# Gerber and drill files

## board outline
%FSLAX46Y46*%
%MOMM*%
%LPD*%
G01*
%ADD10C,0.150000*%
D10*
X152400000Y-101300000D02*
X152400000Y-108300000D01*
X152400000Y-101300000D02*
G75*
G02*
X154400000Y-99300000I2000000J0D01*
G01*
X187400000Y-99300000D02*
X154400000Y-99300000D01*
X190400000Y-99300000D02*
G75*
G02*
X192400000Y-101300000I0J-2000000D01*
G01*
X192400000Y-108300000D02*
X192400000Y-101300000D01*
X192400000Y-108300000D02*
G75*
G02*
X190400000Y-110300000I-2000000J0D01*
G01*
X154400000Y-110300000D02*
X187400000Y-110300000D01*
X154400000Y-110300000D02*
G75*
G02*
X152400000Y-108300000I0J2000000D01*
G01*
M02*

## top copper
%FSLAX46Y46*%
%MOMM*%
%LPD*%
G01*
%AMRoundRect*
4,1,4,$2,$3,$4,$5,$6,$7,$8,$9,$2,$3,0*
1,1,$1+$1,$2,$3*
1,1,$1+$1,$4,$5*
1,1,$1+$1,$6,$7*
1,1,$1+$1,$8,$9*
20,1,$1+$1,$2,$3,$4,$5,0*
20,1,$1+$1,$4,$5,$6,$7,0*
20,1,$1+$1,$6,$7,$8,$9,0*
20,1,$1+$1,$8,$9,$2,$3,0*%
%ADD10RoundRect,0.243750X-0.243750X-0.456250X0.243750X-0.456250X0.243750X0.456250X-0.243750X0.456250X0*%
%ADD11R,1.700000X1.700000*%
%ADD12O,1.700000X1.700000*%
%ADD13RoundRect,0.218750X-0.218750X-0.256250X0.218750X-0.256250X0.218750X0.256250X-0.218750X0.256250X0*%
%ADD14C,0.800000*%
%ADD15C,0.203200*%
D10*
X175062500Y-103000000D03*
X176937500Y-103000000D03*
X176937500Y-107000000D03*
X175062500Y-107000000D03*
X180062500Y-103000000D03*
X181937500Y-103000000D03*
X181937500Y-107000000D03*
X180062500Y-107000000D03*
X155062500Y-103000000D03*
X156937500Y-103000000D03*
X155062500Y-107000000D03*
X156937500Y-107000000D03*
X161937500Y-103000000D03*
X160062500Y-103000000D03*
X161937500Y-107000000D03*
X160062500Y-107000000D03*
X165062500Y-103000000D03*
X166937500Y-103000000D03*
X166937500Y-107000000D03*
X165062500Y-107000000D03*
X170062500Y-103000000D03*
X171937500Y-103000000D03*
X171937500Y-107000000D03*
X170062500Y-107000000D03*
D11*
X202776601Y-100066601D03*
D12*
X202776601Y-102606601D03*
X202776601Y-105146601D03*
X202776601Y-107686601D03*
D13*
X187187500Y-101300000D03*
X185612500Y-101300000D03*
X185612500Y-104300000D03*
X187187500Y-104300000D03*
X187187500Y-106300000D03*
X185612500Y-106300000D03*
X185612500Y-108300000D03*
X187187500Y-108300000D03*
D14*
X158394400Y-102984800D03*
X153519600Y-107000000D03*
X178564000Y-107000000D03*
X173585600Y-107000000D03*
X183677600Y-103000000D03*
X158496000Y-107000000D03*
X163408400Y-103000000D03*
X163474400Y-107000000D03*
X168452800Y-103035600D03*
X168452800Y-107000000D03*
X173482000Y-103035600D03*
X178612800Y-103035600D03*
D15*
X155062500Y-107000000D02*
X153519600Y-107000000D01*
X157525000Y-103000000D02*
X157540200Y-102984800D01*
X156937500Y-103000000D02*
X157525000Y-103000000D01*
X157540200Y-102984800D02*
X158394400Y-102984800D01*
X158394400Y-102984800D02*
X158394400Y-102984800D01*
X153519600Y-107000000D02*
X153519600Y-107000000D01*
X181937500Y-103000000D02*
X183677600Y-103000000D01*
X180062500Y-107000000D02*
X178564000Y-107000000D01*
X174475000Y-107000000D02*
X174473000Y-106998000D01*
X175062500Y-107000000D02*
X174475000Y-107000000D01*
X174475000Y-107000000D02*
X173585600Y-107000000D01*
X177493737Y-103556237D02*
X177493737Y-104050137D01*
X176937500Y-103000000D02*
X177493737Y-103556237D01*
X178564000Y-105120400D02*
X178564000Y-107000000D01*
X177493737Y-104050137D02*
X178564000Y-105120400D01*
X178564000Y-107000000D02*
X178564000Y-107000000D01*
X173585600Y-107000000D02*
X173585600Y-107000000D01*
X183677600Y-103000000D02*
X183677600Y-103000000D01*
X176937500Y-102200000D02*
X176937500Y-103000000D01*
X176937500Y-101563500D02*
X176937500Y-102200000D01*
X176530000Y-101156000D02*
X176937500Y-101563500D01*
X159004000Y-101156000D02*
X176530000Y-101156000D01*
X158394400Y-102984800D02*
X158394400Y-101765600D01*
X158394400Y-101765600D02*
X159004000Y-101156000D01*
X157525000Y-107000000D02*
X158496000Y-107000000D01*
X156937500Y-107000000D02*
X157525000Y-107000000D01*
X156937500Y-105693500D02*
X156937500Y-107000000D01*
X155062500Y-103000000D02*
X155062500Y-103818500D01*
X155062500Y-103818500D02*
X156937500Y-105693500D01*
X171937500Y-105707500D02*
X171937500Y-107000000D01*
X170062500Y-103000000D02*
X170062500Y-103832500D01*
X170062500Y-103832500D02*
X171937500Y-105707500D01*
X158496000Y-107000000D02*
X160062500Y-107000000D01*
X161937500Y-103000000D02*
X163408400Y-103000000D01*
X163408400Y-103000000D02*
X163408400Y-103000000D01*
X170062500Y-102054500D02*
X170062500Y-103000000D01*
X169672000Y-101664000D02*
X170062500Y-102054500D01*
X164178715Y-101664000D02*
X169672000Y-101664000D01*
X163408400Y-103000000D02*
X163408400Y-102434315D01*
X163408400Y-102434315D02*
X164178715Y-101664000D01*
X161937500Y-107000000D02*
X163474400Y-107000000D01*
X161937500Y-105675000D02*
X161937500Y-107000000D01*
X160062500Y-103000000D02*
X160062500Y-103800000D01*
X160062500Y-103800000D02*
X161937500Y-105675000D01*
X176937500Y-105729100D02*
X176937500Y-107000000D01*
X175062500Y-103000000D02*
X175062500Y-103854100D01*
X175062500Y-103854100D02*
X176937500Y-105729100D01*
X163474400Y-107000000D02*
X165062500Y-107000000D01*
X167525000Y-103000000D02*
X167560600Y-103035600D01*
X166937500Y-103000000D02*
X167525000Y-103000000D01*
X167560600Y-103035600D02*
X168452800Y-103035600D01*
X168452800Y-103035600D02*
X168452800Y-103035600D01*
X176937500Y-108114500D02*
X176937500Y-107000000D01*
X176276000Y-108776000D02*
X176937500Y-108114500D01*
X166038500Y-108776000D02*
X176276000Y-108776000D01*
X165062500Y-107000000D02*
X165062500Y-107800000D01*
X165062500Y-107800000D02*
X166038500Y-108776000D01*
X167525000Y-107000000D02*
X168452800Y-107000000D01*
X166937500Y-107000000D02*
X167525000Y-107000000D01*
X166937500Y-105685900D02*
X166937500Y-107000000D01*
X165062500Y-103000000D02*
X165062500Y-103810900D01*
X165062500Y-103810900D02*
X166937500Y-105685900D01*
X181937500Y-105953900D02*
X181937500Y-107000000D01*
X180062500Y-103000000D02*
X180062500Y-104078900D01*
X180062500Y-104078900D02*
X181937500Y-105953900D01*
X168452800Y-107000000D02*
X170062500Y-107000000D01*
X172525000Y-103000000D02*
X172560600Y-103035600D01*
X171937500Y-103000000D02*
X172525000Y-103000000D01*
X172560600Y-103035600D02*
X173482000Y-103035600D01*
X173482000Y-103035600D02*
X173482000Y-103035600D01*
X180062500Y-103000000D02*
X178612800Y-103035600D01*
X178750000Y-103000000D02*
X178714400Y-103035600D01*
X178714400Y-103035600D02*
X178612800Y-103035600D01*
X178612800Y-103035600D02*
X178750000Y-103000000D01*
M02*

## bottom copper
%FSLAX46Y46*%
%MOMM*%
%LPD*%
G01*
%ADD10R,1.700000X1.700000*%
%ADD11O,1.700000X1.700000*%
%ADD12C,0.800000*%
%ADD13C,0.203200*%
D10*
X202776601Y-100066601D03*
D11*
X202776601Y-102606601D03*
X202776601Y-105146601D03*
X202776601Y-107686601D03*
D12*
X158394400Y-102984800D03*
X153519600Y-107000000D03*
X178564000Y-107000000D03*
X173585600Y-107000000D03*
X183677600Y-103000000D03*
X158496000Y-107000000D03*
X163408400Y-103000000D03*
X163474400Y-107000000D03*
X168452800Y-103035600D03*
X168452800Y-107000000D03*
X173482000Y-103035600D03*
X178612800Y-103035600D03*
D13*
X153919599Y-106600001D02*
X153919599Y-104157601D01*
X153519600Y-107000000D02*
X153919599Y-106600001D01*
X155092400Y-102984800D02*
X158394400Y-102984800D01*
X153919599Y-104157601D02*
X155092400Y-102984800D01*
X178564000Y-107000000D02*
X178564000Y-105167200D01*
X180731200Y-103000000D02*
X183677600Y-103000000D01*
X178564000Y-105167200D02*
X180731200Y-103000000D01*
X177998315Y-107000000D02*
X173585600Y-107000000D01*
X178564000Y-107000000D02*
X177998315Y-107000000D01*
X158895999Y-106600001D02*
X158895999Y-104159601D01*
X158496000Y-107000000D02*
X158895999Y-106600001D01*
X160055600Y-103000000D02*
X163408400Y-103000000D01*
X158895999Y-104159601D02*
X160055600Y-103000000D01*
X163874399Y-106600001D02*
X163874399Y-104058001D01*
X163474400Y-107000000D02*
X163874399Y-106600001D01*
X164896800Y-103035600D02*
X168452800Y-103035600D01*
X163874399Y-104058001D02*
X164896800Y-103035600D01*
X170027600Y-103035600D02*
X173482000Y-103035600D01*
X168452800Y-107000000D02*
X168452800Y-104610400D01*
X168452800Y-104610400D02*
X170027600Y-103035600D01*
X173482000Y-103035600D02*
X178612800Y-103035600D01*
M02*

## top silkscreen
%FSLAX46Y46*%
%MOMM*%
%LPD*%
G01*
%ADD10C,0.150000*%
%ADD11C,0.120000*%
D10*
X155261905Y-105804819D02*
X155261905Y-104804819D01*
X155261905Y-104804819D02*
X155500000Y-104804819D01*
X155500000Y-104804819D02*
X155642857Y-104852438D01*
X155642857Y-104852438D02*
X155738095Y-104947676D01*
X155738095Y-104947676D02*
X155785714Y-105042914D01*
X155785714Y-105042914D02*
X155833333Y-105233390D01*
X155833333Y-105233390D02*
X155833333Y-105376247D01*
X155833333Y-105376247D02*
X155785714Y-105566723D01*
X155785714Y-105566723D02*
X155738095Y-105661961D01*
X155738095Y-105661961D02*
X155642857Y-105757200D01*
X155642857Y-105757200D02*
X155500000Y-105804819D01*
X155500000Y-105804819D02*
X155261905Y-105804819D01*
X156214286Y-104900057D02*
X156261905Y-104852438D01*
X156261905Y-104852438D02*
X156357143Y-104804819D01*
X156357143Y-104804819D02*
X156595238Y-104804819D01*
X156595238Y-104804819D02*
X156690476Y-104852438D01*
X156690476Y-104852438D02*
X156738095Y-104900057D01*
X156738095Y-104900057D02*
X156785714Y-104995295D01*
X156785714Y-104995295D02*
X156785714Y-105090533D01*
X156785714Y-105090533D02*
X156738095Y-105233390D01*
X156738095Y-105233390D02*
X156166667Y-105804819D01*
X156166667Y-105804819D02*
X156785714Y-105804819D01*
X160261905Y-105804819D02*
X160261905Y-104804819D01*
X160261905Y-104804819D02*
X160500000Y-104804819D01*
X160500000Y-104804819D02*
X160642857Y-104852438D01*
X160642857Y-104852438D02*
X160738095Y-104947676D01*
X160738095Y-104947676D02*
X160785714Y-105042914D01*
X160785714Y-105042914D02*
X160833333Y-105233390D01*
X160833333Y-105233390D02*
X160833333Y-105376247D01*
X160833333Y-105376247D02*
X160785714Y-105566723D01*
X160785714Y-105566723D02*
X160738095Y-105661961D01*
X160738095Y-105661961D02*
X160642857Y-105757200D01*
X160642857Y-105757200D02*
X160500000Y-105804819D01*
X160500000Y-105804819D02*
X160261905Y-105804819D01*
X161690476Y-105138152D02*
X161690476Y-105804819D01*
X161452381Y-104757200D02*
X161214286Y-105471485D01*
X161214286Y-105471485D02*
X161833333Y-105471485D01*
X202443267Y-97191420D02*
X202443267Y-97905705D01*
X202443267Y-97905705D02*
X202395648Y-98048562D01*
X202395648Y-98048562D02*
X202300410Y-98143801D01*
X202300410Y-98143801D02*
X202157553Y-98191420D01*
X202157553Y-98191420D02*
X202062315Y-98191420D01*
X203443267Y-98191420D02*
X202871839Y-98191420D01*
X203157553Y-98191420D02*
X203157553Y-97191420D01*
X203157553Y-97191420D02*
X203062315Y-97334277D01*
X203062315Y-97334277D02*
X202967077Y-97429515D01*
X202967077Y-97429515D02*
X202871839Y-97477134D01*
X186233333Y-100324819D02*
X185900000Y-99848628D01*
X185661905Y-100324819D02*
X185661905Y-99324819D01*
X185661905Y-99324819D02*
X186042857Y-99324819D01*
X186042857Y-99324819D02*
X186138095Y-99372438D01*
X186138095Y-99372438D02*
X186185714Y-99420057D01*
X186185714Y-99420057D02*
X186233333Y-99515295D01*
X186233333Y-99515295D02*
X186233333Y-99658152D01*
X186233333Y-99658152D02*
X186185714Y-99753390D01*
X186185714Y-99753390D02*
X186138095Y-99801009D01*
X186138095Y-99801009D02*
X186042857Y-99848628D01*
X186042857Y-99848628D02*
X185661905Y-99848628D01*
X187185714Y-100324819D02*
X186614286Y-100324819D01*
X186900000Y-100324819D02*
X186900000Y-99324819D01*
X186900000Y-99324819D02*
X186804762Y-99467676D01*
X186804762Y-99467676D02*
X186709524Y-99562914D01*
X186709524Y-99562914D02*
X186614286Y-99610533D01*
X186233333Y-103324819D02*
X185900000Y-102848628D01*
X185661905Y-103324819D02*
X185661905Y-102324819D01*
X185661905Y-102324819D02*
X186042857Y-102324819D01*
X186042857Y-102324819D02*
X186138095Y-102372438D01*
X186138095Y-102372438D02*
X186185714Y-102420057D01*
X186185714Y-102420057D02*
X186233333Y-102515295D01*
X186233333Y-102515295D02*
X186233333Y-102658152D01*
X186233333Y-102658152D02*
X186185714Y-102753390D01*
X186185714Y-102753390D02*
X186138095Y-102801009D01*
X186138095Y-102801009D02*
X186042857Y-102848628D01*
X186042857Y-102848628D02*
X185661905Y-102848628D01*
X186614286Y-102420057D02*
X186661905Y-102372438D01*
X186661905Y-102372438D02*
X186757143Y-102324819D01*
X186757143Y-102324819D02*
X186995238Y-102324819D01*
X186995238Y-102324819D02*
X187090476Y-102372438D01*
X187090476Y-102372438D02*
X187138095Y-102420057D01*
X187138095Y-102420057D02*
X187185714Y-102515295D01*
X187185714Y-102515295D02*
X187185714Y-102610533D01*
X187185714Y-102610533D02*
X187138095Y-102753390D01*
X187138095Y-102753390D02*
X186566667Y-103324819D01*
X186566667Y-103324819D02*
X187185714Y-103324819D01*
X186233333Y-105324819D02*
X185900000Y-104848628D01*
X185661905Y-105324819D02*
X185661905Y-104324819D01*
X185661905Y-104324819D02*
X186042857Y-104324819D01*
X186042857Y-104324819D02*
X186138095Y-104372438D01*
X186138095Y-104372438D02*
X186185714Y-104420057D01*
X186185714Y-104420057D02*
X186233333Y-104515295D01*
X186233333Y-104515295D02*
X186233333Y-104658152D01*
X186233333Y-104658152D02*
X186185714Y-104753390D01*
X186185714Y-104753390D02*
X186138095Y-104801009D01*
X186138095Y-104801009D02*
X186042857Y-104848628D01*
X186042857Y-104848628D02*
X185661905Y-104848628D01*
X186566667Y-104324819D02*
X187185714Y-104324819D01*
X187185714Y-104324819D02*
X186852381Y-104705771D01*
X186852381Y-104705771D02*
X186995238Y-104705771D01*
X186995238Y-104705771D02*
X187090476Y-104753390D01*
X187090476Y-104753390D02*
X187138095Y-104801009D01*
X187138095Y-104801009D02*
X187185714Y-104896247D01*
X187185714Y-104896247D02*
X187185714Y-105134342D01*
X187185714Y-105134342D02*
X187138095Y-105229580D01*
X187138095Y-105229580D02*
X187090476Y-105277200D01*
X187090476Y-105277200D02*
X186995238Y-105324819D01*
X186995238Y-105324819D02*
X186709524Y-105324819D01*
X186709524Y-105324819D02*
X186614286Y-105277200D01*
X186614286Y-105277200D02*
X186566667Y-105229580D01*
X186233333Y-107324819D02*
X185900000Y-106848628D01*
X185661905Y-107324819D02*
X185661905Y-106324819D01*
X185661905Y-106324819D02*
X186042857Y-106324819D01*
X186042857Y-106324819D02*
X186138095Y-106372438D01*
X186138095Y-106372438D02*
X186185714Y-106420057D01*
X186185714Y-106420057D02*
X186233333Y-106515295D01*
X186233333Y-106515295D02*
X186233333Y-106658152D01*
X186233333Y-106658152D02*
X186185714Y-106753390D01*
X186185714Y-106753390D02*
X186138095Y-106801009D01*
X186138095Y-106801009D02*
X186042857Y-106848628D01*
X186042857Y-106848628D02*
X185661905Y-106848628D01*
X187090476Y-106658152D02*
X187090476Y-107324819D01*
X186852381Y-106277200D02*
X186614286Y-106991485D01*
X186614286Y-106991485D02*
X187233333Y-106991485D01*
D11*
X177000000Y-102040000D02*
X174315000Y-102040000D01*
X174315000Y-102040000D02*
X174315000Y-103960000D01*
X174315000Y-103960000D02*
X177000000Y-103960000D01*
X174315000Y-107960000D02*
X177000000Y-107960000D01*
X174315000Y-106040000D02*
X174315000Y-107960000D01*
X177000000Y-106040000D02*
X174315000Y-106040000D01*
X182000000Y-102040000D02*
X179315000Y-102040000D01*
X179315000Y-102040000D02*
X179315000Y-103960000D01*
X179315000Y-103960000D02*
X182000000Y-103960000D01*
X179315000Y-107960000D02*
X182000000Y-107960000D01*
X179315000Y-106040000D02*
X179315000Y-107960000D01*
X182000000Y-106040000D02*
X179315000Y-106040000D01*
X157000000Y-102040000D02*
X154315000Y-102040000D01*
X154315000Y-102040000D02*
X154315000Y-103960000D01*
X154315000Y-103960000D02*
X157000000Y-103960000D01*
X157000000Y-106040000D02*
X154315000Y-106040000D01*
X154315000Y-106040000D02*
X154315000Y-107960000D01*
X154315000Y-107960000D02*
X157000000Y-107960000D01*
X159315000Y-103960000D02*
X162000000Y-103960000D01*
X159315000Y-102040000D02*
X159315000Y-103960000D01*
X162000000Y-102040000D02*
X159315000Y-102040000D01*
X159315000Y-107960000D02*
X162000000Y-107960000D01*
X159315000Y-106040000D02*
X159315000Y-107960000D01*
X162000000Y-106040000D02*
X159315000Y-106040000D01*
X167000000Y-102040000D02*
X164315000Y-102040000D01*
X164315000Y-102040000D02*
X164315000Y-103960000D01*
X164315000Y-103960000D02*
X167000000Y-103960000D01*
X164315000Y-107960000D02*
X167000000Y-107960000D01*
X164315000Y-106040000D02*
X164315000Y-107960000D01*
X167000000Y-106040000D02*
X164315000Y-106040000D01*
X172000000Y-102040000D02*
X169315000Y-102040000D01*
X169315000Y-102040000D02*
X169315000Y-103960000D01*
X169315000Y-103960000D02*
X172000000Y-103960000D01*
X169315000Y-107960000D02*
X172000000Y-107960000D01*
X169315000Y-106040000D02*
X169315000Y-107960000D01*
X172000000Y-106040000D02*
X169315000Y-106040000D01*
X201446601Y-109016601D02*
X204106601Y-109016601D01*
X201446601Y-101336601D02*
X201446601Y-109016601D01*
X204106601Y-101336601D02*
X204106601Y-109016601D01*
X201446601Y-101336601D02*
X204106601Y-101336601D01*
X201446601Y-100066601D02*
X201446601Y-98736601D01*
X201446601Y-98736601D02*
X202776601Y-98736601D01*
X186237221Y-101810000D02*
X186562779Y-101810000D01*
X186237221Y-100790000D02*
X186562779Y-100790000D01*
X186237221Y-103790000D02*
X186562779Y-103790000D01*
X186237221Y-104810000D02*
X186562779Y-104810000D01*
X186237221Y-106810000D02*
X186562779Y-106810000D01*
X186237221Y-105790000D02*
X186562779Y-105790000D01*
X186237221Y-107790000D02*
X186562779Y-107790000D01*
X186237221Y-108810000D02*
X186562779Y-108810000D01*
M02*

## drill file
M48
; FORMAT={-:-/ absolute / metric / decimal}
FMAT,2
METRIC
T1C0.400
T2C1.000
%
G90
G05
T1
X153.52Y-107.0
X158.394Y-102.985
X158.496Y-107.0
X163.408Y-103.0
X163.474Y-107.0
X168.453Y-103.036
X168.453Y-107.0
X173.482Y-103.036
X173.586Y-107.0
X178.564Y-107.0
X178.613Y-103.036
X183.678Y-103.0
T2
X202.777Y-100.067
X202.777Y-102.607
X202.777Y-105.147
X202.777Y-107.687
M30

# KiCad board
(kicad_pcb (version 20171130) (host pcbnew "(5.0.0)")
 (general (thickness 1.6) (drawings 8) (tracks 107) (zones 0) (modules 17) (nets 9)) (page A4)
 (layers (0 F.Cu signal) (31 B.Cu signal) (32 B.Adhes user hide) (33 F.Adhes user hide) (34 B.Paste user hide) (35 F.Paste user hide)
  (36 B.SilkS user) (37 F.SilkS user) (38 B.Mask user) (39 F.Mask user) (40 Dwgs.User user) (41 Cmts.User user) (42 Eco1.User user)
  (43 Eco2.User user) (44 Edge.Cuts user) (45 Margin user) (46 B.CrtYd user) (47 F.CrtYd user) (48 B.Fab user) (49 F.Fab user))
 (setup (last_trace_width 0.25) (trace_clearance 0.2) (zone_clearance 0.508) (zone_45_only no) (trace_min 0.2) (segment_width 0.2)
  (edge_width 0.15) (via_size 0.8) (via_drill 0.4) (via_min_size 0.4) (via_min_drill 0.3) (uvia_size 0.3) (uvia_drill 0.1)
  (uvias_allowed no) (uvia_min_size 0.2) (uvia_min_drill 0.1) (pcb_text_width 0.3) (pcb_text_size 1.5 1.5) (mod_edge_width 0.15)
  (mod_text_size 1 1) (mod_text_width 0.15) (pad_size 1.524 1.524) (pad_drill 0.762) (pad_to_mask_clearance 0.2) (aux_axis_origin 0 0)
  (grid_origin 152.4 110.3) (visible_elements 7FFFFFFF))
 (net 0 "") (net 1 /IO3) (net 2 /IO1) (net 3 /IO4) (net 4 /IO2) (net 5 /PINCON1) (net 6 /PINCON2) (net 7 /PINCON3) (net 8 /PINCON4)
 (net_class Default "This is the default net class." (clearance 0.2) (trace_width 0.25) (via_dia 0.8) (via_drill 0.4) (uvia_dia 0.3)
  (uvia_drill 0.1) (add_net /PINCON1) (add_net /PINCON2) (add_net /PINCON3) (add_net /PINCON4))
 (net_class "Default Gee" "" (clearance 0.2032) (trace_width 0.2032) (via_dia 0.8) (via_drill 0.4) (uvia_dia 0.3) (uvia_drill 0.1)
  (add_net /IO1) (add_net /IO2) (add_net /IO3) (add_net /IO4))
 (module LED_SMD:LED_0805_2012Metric (layer F.Cu) (at 176 103)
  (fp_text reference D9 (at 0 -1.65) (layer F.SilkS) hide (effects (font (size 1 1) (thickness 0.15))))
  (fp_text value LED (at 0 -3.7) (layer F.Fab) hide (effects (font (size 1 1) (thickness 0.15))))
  (fp_line (start 1 -0.96) (end -1.685 -0.96) (layer F.SilkS) (width 0.12))
  (fp_line (start -1.685 -0.96) (end -1.685 0.96) (layer F.SilkS) (width 0.12))
  (fp_line (start -1.685 0.96) (end 1 0.96) (layer F.SilkS) (width 0.12))
  (pad 1 smd roundrect (at -0.9375 0) (size 0.975 1.4) (layers F.Cu F.Paste F.Mask) (roundrect_rratio 0.25) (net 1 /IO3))
  (pad 2 smd roundrect (at 0.9375 0) (size 0.975 1.4) (layers F.Cu F.Paste F.Mask) (roundrect_rratio 0.25) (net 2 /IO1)))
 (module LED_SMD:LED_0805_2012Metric (layer F.Cu) (at 176 107)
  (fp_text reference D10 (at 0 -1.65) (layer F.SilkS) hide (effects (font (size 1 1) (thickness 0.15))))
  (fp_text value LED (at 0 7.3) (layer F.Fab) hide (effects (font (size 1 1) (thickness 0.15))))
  (fp_line (start -1.685 0.96) (end 1 0.96) (layer F.SilkS) (width 0.12))
  (fp_line (start -1.685 -0.96) (end -1.685 0.96) (layer F.SilkS) (width 0.12))
  (fp_line (start 1 -0.96) (end -1.685 -0.96) (layer F.SilkS) (width 0.12))
  (pad 2 smd roundrect (at 0.9375 0) (size 0.975 1.4) (layers F.Cu F.Paste F.Mask) (roundrect_rratio 0.25) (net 1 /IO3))
  (pad 1 smd roundrect (at -0.9375 0) (size 0.975 1.4) (layers F.Cu F.Paste F.Mask) (roundrect_rratio 0.25) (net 2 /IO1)))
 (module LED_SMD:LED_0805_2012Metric (layer F.Cu) (at 181 103)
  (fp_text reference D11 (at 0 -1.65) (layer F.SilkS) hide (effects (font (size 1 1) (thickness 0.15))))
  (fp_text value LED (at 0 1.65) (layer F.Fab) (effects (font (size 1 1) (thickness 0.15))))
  (fp_line (start 1 -0.96) (end -1.685 -0.96) (layer F.SilkS) (width 0.12))
  (fp_line (start -1.685 -0.96) (end -1.685 0.96) (layer F.SilkS) (width 0.12))
  (fp_line (start -1.685 0.96) (end 1 0.96) (layer F.SilkS) (width 0.12))
  (pad 1 smd roundrect (at -0.9375 0) (size 0.975 1.4) (layers F.Cu F.Paste F.Mask) (roundrect_rratio 0.25) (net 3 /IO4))
  (pad 2 smd roundrect (at 0.9375 0) (size 0.975 1.4) (layers F.Cu F.Paste F.Mask) (roundrect_rratio 0.25) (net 2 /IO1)))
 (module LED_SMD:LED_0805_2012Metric (layer F.Cu) (at 181 107)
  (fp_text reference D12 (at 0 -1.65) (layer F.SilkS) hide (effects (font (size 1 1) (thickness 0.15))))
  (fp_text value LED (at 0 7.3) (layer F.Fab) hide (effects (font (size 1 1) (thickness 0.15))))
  (fp_line (start -1.685 0.96) (end 1 0.96) (layer F.SilkS) (width 0.12))
  (fp_line (start -1.685 -0.96) (end -1.685 0.96) (layer F.SilkS) (width 0.12))
  (fp_line (start 1 -0.96) (end -1.685 -0.96) (layer F.SilkS) (width 0.12))
  (pad 2 smd roundrect (at 0.9375 0) (size 0.975 1.4) (layers F.Cu F.Paste F.Mask) (roundrect_rratio 0.25) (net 3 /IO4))
  (pad 1 smd roundrect (at -0.9375 0) (size 0.975 1.4) (layers F.Cu F.Paste F.Mask) (roundrect_rratio 0.25) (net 2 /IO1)))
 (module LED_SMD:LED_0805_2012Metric (layer F.Cu) (at 156 103)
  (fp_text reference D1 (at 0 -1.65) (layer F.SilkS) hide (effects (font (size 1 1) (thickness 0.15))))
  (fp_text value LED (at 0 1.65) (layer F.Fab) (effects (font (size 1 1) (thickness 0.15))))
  (fp_line (start 1 -0.96) (end -1.685 -0.96) (layer F.SilkS) (width 0.12))
  (fp_line (start -1.685 -0.96) (end -1.685 0.96) (layer F.SilkS) (width 0.12))
  (fp_line (start -1.685 0.96) (end 1 0.96) (layer F.SilkS) (width 0.12))
  (pad 1 smd roundrect (at -0.9375 0) (size 0.975 1.4) (layers F.Cu F.Paste F.Mask) (roundrect_rratio 0.25) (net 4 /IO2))
  (pad 2 smd roundrect (at 0.9375 0) (size 0.975 1.4) (layers F.Cu F.Paste F.Mask) (roundrect_rratio 0.25) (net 2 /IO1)))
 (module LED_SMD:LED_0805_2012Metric (layer F.Cu) (at 156 107)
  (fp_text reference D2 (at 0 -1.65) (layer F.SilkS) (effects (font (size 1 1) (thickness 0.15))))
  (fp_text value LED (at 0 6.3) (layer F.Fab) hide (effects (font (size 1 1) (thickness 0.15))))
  (fp_line (start 1 -0.96) (end -1.685 -0.96) (layer F.SilkS) (width 0.12))
  (fp_line (start -1.685 -0.96) (end -1.685 0.96) (layer F.SilkS) (width 0.12))
  (fp_line (start -1.685 0.96) (end 1 0.96) (layer F.SilkS) (width 0.12))
  (pad 1 smd roundrect (at -0.9375 0) (size 0.975 1.4) (layers F.Cu F.Paste F.Mask) (roundrect_rratio 0.25) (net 2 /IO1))
  (pad 2 smd roundrect (at 0.9375 0) (size 0.975 1.4) (layers F.Cu F.Paste F.Mask) (roundrect_rratio 0.25) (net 4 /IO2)))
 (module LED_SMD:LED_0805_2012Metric (layer F.Cu) (at 161 103)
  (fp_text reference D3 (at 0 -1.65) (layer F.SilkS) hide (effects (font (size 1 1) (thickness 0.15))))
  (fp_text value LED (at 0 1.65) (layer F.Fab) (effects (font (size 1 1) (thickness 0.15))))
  (fp_line (start -1.685 0.96) (end 1 0.96) (layer F.SilkS) (width 0.12))
  (fp_line (start -1.685 -0.96) (end -1.685 0.96) (layer F.SilkS) (width 0.12))
  (fp_line (start 1 -0.96) (end -1.685 -0.96) (layer F.SilkS) (width 0.12))
  (pad 2 smd roundrect (at 0.9375 0) (size 0.975 1.4) (layers F.Cu F.Paste F.Mask) (roundrect_rratio 0.25) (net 4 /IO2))
  (pad 1 smd roundrect (at -0.9375 0) (size 0.975 1.4) (layers F.Cu F.Paste F.Mask) (roundrect_rratio 0.25) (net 1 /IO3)))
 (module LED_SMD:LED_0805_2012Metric (layer F.Cu) (at 161 107)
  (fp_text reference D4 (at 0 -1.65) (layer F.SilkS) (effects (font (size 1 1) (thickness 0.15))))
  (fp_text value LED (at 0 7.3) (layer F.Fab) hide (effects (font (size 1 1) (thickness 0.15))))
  (fp_line (start -1.685 0.96) (end 1 0.96) (layer F.SilkS) (width 0.12))
  (fp_line (start -1.685 -0.96) (end -1.685 0.96) (layer F.SilkS) (width 0.12))
  (fp_line (start 1 -0.96) (end -1.685 -0.96) (layer F.SilkS) (width 0.12))
  (pad 2 smd roundrect (at 0.9375 0) (size 0.975 1.4) (layers F.Cu F.Paste F.Mask) (roundrect_rratio 0.25) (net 1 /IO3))
  (pad 1 smd roundrect (at -0.9375 0) (size 0.975 1.4) (layers F.Cu F.Paste F.Mask) (roundrect_rratio 0.25) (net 4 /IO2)))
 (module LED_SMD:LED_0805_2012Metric (layer F.Cu) (at 166 103)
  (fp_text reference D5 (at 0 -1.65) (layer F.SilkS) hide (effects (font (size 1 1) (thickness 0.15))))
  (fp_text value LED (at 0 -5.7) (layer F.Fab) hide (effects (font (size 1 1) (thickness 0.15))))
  (fp_line (start 1 -0.96) (end -1.685 -0.96) (layer F.SilkS) (width 0.12))
  (fp_line (start -1.685 -0.96) (end -1.685 0.96) (layer F.SilkS) (width 0.12))
  (fp_line (start -1.685 0.96) (end 1 0.96) (layer F.SilkS) (width 0.12))
  (pad 1 smd roundrect (at -0.9375 0) (size 0.975 1.4) (layers F.Cu F.Paste F.Mask) (roundrect_rratio 0.25) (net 3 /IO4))
  (pad 2 smd roundrect (at 0.9375 0) (size 0.975 1.4) (layers F.Cu F.Paste F.Mask) (roundrect_rratio 0.25) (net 1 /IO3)))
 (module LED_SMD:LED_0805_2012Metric (layer F.Cu) (at 166 107)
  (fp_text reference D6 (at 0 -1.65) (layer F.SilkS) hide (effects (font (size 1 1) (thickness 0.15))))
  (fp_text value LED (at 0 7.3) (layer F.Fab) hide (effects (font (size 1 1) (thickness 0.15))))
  (fp_line (start -1.685 0.96) (end 1 0.96) (layer F.SilkS) (width 0.12))
  (fp_line (start -1.685 -0.96) (end -1.685 0.96) (layer F.SilkS) (width 0.12))
  (fp_line (start 1 -0.96) (end -1.685 -0.96) (layer F.SilkS) (width 0.12))
  (pad 2 smd roundrect (at 0.9375 0) (size 0.975 1.4) (layers F.Cu F.Paste F.Mask) (roundrect_rratio 0.25) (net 3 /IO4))
  (pad 1 smd roundrect (at -0.9375 0) (size 0.975 1.4) (layers F.Cu F.Paste F.Mask) (roundrect_rratio 0.25) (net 1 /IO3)))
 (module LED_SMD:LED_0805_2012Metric (layer F.Cu) (at 171 103)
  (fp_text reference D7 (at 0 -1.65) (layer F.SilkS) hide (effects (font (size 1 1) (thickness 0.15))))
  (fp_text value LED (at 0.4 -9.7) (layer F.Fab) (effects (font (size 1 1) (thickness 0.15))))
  (fp_line (start 1 -0.96) (end -1.685 -0.96) (layer F.SilkS) (width 0.12))
  (fp_line (start -1.685 -0.96) (end -1.685 0.96) (layer F.SilkS) (width 0.12))
  (fp_line (start -1.685 0.96) (end 1 0.96) (layer F.SilkS) (width 0.12))
  (pad 1 smd roundrect (at -0.9375 0) (size 0.975 1.4) (layers F.Cu F.Paste F.Mask) (roundrect_rratio 0.25) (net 4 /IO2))
  (pad 2 smd roundrect (at 0.9375 0) (size 0.975 1.4) (layers F.Cu F.Paste F.Mask) (roundrect_rratio 0.25) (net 3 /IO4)))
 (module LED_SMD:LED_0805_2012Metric (layer F.Cu) (at 171 107)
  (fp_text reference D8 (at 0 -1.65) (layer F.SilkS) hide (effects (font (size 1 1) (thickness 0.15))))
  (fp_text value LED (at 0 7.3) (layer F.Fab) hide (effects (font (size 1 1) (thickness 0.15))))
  (fp_line (start -1.685 0.96) (end 1 0.96) (layer F.SilkS) (width 0.12))
  (fp_line (start -1.685 -0.96) (end -1.685 0.96) (layer F.SilkS) (width 0.12))
  (fp_line (start 1 -0.96) (end -1.685 -0.96) (layer F.SilkS) (width 0.12))
  (pad 2 smd roundrect (at 0.9375 0) (size 0.975 1.4) (layers F.Cu F.Paste F.Mask) (roundrect_rratio 0.25) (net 4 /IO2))
  (pad 1 smd roundrect (at -0.9375 0) (size 0.975 1.4) (layers F.Cu F.Paste F.Mask) (roundrect_rratio 0.25) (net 3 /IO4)))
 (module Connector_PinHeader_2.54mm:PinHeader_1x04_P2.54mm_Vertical (layer F.Cu) (at 202.776601 100.066601)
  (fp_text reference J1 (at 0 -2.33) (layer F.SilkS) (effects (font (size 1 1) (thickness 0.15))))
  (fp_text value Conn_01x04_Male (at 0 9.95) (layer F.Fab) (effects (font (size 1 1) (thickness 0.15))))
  (fp_line (start -1.33 8.95) (end 1.33 8.95) (layer F.SilkS) (width 0.12))
  (fp_line (start -1.33 1.27) (end -1.33 8.95) (layer F.SilkS) (width 0.12))
  (fp_line (start 1.33 1.27) (end 1.33 8.95) (layer F.SilkS) (width 0.12))
  (fp_line (start -1.33 1.27) (end 1.33 1.27) (layer F.SilkS) (width 0.12))
  (fp_line (start -1.33 0) (end -1.33 -1.33) (layer F.SilkS) (width 0.12))
  (fp_line (start -1.33 -1.33) (end 0 -1.33) (layer F.SilkS) (width 0.12))
  (pad 1 thru_hole rect (at 0 0) (size 1.7 1.7) (drill 1) (layers *.Cu *.Mask) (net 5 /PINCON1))
  (pad 2 thru_hole oval (at 0 2.54) (size 1.7 1.7) (drill 1) (layers *.Cu *.Mask) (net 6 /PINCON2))
  (pad 3 thru_hole oval (at 0 5.08) (size 1.7 1.7) (drill 1) (layers *.Cu *.Mask) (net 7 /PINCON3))
  (pad 4 thru_hole oval (at 0 7.62) (size 1.7 1.7) (drill 1) (layers *.Cu *.Mask) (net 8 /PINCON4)))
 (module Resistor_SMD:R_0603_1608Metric (layer F.Cu) (at 186.4 101.3)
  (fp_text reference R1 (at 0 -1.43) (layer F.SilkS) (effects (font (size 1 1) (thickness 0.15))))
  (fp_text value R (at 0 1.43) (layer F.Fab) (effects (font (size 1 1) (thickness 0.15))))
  (fp_line (start -0.162779 0.51) (end 0.162779 0.51) (layer F.SilkS) (width 0.12))
  (fp_line (start -0.162779 -0.51) (end 0.162779 -0.51) (layer F.SilkS) (width 0.12))
  (pad 2 smd roundrect (at 0.7875 0) (size 0.875 0.95) (layers F.Cu F.Paste F.Mask) (roundrect_rratio 0.25) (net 2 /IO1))
  (pad 1 smd roundrect (at -0.7875 0) (size 0.875 0.95) (layers F.Cu F.Paste F.Mask) (roundrect_rratio 0.25) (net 5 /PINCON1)))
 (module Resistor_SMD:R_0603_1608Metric (layer F.Cu) (at 186.4 104.3)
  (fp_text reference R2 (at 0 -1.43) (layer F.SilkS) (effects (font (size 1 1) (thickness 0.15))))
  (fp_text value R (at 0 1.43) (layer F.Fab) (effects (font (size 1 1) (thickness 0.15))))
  (fp_line (start -0.162779 -0.51) (end 0.162779 -0.51) (layer F.SilkS) (width 0.12))
  (fp_line (start -0.162779 0.51) (end 0.162779 0.51) (layer F.SilkS) (width 0.12))
  (pad 1 smd roundrect (at -0.7875 0) (size 0.875 0.95) (layers F.Cu F.Paste F.Mask) (roundrect_rratio 0.25) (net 6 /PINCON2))
  (pad 2 smd roundrect (at 0.7875 0) (size 0.875 0.95) (layers F.Cu F.Paste F.Mask) (roundrect_rratio 0.25) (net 4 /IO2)))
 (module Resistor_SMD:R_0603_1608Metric (layer F.Cu) (at 186.4 106.3)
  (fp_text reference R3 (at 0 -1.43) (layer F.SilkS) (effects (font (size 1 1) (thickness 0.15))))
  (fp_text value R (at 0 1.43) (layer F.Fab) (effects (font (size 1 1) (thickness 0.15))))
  (fp_line (start -0.162779 0.51) (end 0.162779 0.51) (layer F.SilkS) (width 0.12))
  (fp_line (start -0.162779 -0.51) (end 0.162779 -0.51) (layer F.SilkS) (width 0.12))
  (pad 2 smd roundrect (at 0.7875 0) (size 0.875 0.95) (layers F.Cu F.Paste F.Mask) (roundrect_rratio 0.25) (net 1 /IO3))
  (pad 1 smd roundrect (at -0.7875 0) (size 0.875 0.95) (layers F.Cu F.Paste F.Mask) (roundrect_rratio 0.25) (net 7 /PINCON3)))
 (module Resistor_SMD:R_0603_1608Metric (layer F.Cu) (at 186.4 108.3)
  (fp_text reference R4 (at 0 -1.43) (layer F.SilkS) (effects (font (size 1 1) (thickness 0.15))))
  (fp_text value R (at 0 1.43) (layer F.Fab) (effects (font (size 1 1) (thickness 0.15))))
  (fp_line (start -0.162779 -0.51) (end 0.162779 -0.51) (layer F.SilkS) (width 0.12))
  (fp_line (start -0.162779 0.51) (end 0.162779 0.51) (layer F.SilkS) (width 0.12))
  (pad 1 smd roundrect (at -0.7875 0) (size 0.875 0.95) (layers F.Cu F.Paste F.Mask) (roundrect_rratio 0.25) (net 8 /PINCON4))
  (pad 2 smd roundrect (at 0.7875 0) (size 0.875 0.95) (layers F.Cu F.Paste F.Mask) (roundrect_rratio 0.25) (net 3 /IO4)))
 (gr_line (start 152.4 101.3) (end 152.4 108.3) (layer Edge.Cuts) (width 0.15))
 (gr_arc (start 154.4 101.3) (end 154.4 99.3) (angle -90) (layer Edge.Cuts) (width 0.15))
 (gr_line (start 187.4 99.3) (end 154.4 99.3) (layer Edge.Cuts) (width 0.15))
 (gr_arc (start 190.4 101.3) (end 192.4 101.3) (angle -90) (layer Edge.Cuts) (width 0.15))
 (gr_line (start 192.4 108.3) (end 192.4 101.3) (layer Edge.Cuts) (width 0.15))
 (gr_arc (start 190.4 108.3) (end 190.4 110.3) (angle -90) (layer Edge.Cuts) (width 0.15))
 (gr_line (start 154.4 110.3) (end 187.4 110.3) (layer Edge.Cuts) (width 0.15))
 (gr_arc (start 154.4 108.3) (end 152.4 108.3) (angle -90) (layer Edge.Cuts) (width 0.15))
 (segment (start 155.0625 107) (end 153.5196 107) (width 0.2032) (layer F.Cu) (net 2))
 (segment (start 157.525 103) (end 157.5402 102.9848) (width 0.2032) (layer F.Cu) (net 2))
 (segment (start 156.9375 103) (end 157.525 103) (width 0.2032) (layer F.Cu) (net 2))
 (segment (start 157.5402 102.9848) (end 158.3944 102.9848) (width 0.2032) (layer F.Cu) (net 2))
 (segment (start 158.3944 102.9848) (end 158.3944 102.9848) (width 0.2032) (layer F.Cu) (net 2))
 (via (at 158.3944 102.9848) (size 0.8) (drill 0.4) (layers F.Cu B.Cu) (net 2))
 (segment (start 153.5196 107) (end 153.5196 107) (width 0.2032) (layer F.Cu) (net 2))
 (via (at 153.5196 107) (size 0.8) (drill 0.4) (layers F.Cu B.Cu) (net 2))
 (segment (start 153.919599 106.600001) (end 153.919599 104.157601) (width 0.2032) (layer B.Cu) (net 2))
 (segment (start 153.5196 107) (end 153.919599 106.600001) (width 0.2032) (layer B.Cu) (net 2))
 (segment (start 155.0924 102.9848) (end 158.3944 102.9848) (width 0.2032) (layer B.Cu) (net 2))
 (segment (start 153.919599 104.157601) (end 155.0924 102.9848) (width 0.2032) (layer B.Cu) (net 2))
 (segment (start 181.9375 103) (end 183.6776 103) (width 0.2032) (layer F.Cu) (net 2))
 (segment (start 180.0625 107) (end 178.564 107) (width 0.2032) (layer F.Cu) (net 2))
 (segment (start 174.475 107) (end 174.473 106.998) (width 0.2032) (layer F.Cu) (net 2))
 (segment (start 175.0625 107) (end 174.475 107) (width 0.2032) (layer F.Cu) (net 2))
 (segment (start 174.475 107) (end 173.5856 107) (width 0.2032) (layer F.Cu) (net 2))
 (segment (start 177.493737 103.556237) (end 177.493737 104.050137) (width 0.2032) (layer F.Cu) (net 2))
 (segment (start 176.9375 103) (end 177.493737 103.556237) (width 0.2032) (layer F.Cu) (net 2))
 (segment (start 178.564 105.1204) (end 178.564 107) (width 0.2032) (layer F.Cu) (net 2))
 (segment (start 177.493737 104.050137) (end 178.564 105.1204) (width 0.2032) (layer F.Cu) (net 2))
 (segment (start 178.564 107) (end 178.564 107) (width 0.2032) (layer F.Cu) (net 2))
 (via (at 178.564 107) (size 0.8) (drill 0.4) (layers F.Cu B.Cu) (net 2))
 (segment (start 173.5856 107) (end 173.5856 107) (width 0.2032) (layer F.Cu) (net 2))
 (via (at 173.5856 107) (size 0.8) (drill 0.4) (layers F.Cu B.Cu) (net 2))
 (segment (start 183.6776 103) (end 183.6776 103) (width 0.2032) (layer F.Cu) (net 2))
 (via (at 183.6776 103) (size 0.8) (drill 0.4) (layers F.Cu B.Cu) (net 2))
 (segment (start 178.564 107) (end 178.564 105.1672) (width 0.2032) (layer B.Cu) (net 2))
 (segment (start 180.7312 103) (end 183.6776 103) (width 0.2032) (layer B.Cu) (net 2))
 (segment (start 178.564 105.1672) (end 180.7312 103) (width 0.2032) (layer B.Cu) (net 2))
 (segment (start 176.9375 102.2) (end 176.9375 103) (width 0.2032) (layer F.Cu) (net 2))
 (segment (start 176.9375 101.5635) (end 176.9375 102.2) (width 0.2032) (layer F.Cu) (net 2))
 (segment (start 176.53 101.156) (end 176.9375 101.5635) (width 0.2032) (layer F.Cu) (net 2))
 (segment (start 159.004 101.156) (end 176.53 101.156) (width 0.2032) (layer F.Cu) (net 2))
 (segment (start 158.3944 102.9848) (end 158.3944 101.7656) (width 0.2032) (layer F.Cu) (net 2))
 (segment (start 158.3944 101.7656) (end 159.004 101.156) (width 0.2032) (layer F.Cu) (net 2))
 (segment (start 177.998315 107) (end 173.5856 107) (width 0.2032) (layer B.Cu) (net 2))
 (segment (start 178.564 107) (end 177.998315 107) (width 0.2032) (layer B.Cu) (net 2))
 (segment (start 157.525 107) (end 158.496 107) (width 0.2032) (layer F.Cu) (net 4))
 (segment (start 156.9375 107) (end 157.525 107) (width 0.2032) (layer F.Cu) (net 4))
 (segment (start 156.9375 105.6935) (end 156.9375 107) (width 0.2032) (layer F.Cu) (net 4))
 (segment (start 155.0625 103) (end 155.0625 103.8185) (width 0.2032) (layer F.Cu) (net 4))
 (segment (start 155.0625 103.8185) (end 156.9375 105.6935) (width 0.2032) (layer F.Cu) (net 4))
 (segment (start 171.9375 105.7075) (end 171.9375 107) (width 0.2032) (layer F.Cu) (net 4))
 (segment (start 170.0625 103) (end 170.0625 103.8325) (width 0.2032) (layer F.Cu) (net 4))
 (segment (start 170.0625 103.8325) (end 171.9375 105.7075) (width 0.2032) (layer F.Cu) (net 4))
 (segment (start 158.496 107) (end 160.0625 107) (width 0.2032) (layer F.Cu) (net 4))
 (via (at 158.496 107) (size 0.8) (drill 0.4) (layers F.Cu B.Cu) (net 4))
 (segment (start 161.9375 103) (end 163.4084 103) (width 0.2032) (layer F.Cu) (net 4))
 (segment (start 163.4084 103) (end 163.4084 103) (width 0.2032) (layer F.Cu) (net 4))
 (via (at 163.4084 103) (size 0.8) (drill 0.4) (layers F.Cu B.Cu) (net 4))
 (segment (start 158.895999 106.600001) (end 158.895999 104.159601) (width 0.2032) (layer B.Cu) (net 4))
 (segment (start 158.496 107) (end 158.895999 106.600001) (width 0.2032) (layer B.Cu) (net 4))
 (segment (start 160.0556 103) (end 163.4084 103) (width 0.2032) (layer B.Cu) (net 4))
 (segment (start 158.895999 104.159601) (end 160.0556 103) (width 0.2032) (layer B.Cu) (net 4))
 (segment (start 170.0625 102.0545) (end 170.0625 103) (width 0.2032) (layer F.Cu) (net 4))
 (segment (start 169.672 101.664) (end 170.0625 102.0545) (width 0.2032) (layer F.Cu) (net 4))
 (segment (start 164.178715 101.664) (end 169.672 101.664) (width 0.2032) (layer F.Cu) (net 4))
 (segment (start 163.4084 103) (end 163.4084 102.434315) (width 0.2032) (layer F.Cu) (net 4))
 (segment (start 163.4084 102.434315) (end 164.178715 101.664) (width 0.2032) (layer F.Cu) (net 4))
 (segment (start 161.9375 107) (end 163.4744 107) (width 0.2032) (layer F.Cu) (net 1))
 (segment (start 161.9375 105.675) (end 161.9375 107) (width 0.2032) (layer F.Cu) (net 1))
 (segment (start 160.0625 103) (end 160.0625 103.8) (width 0.2032) (layer F.Cu) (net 1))
 (segment (start 160.0625 103.8) (end 161.9375 105.675) (width 0.2032) (layer F.Cu) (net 1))
 (segment (start 176.9375 105.7291) (end 176.9375 107) (width 0.2032) (layer F.Cu) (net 1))
 (segment (start 175.0625 103) (end 175.0625 103.8541) (width 0.2032) (layer F.Cu) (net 1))
 (segment (start 175.0625 103.8541) (end 176.9375 105.7291) (width 0.2032) (layer F.Cu) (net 1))
 (segment (start 163.4744 107) (end 165.0625 107) (width 0.2032) (layer F.Cu) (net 1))
 (via (at 163.4744 107) (size 0.8) (drill 0.4) (layers F.Cu B.Cu) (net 1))
 (segment (start 167.525 103) (end 167.5606 103.0356) (width 0.2032) (layer F.Cu) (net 1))
 (segment (start 166.9375 103) (end 167.525 103) (width 0.2032) (layer F.Cu) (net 1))
 (segment (start 167.5606 103.0356) (end 168.4528 103.0356) (width 0.2032) (layer F.Cu) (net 1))
 (segment (start 168.4528 103.0356) (end 168.4528 103.0356) (width 0.2032) (layer F.Cu) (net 1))
 (via (at 168.4528 103.0356) (size 0.8) (drill 0.4) (layers F.Cu B.Cu) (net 1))
 (segment (start 163.874399 106.600001) (end 163.874399 104.058001) (width 0.2032) (layer B.Cu) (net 1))
 (segment (start 163.4744 107) (end 163.874399 106.600001) (width 0.2032) (layer B.Cu) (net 1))
 (segment (start 164.8968 103.0356) (end 168.4528 103.0356) (width 0.2032) (layer B.Cu) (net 1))
 (segment (start 163.874399 104.058001) (end 164.8968 103.0356) (width 0.2032) (layer B.Cu) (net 1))
 (segment (start 176.9375 108.1145) (end 176.9375 107) (width 0.2032) (layer F.Cu) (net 1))
 (segment (start 176.276 108.776) (end 176.9375 108.1145) (width 0.2032) (layer F.Cu) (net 1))
 (segment (start 166.0385 108.776) (end 176.276 108.776) (width 0.2032) (layer F.Cu) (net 1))
 (segment (start 165.0625 107) (end 165.0625 107.8) (width 0.2032) (layer F.Cu) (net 1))
 (segment (start 165.0625 107.8) (end 166.0385 108.776) (width 0.2032) (layer F.Cu) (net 1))
 (segment (start 167.525 107) (end 168.4528 107) (width 0.2032) (layer F.Cu) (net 3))
 (segment (start 166.9375 107) (end 167.525 107) (width 0.2032) (layer F.Cu) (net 3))
 (segment (start 166.9375 105.6859) (end 166.9375 107) (width 0.2032) (layer F.Cu) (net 3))
 (segment (start 165.0625 103) (end 165.0625 103.8109) (width 0.2032) (layer F.Cu) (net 3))
 (segment (start 165.0625 103.8109) (end 166.9375 105.6859) (width 0.2032) (layer F.Cu) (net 3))
 (segment (start 181.9375 105.9539) (end 181.9375 107) (width 0.2032) (layer F.Cu) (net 3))
 (segment (start 180.0625 103) (end 180.0625 104.0789) (width 0.2032) (layer F.Cu) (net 3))
 (segment (start 180.0625 104.0789) (end 181.9375 105.9539) (width 0.2032) (layer F.Cu) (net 3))
 (segment (start 168.4528 107) (end 170.0625 107) (width 0.2032) (layer F.Cu) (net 3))
 (via (at 168.4528 107) (size 0.8) (drill 0.4) (layers F.Cu B.Cu) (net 3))
 (segment (start 172.525 103) (end 172.5606 103.0356) (width 0.2032) (layer F.Cu) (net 3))
 (segment (start 171.9375 103) (end 172.525 103) (width 0.2032) (layer F.Cu) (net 3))
 (segment (start 172.5606 103.0356) (end 173.482 103.0356) (width 0.2032) (layer F.Cu) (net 3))
 (segment (start 173.482 103.0356) (end 173.482 103.0356) (width 0.2032) (layer F.Cu) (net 3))
 (via (at 173.482 103.0356) (size 0.8) (drill 0.4) (layers F.Cu B.Cu) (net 3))
 (segment (start 170.0276 103.0356) (end 173.482 103.0356) (width 0.2032) (layer B.Cu) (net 3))
 (segment (start 168.4528 107) (end 168.4528 104.6104) (width 0.2032) (layer B.Cu) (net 3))
 (segment (start 168.4528 104.6104) (end 170.0276 103.0356) (width 0.2032) (layer B.Cu) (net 3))
 (segment (start 180.0625 103) (end 178.6128 103.0356) (width 0.2032) (layer F.Cu) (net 3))
 (segment (start 178.75 103) (end 178.7144 103.0356) (width 0.2032) (layer F.Cu) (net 3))
 (segment (start 178.7144 103.0356) (end 178.6128 103.0356) (width 0.2032) (layer F.Cu) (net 3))
 (segment (start 178.6128 103.0356) (end 178.75 103) (width 0.2032) (layer F.Cu) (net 3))
 (via (at 178.6128 103.0356) (size 0.8) (drill 0.4) (layers F.Cu B.Cu) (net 3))
 (segment (start 173.482 103.0356) (end 178.6128 103.0356) (width 0.2032) (layer B.Cu) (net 3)))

